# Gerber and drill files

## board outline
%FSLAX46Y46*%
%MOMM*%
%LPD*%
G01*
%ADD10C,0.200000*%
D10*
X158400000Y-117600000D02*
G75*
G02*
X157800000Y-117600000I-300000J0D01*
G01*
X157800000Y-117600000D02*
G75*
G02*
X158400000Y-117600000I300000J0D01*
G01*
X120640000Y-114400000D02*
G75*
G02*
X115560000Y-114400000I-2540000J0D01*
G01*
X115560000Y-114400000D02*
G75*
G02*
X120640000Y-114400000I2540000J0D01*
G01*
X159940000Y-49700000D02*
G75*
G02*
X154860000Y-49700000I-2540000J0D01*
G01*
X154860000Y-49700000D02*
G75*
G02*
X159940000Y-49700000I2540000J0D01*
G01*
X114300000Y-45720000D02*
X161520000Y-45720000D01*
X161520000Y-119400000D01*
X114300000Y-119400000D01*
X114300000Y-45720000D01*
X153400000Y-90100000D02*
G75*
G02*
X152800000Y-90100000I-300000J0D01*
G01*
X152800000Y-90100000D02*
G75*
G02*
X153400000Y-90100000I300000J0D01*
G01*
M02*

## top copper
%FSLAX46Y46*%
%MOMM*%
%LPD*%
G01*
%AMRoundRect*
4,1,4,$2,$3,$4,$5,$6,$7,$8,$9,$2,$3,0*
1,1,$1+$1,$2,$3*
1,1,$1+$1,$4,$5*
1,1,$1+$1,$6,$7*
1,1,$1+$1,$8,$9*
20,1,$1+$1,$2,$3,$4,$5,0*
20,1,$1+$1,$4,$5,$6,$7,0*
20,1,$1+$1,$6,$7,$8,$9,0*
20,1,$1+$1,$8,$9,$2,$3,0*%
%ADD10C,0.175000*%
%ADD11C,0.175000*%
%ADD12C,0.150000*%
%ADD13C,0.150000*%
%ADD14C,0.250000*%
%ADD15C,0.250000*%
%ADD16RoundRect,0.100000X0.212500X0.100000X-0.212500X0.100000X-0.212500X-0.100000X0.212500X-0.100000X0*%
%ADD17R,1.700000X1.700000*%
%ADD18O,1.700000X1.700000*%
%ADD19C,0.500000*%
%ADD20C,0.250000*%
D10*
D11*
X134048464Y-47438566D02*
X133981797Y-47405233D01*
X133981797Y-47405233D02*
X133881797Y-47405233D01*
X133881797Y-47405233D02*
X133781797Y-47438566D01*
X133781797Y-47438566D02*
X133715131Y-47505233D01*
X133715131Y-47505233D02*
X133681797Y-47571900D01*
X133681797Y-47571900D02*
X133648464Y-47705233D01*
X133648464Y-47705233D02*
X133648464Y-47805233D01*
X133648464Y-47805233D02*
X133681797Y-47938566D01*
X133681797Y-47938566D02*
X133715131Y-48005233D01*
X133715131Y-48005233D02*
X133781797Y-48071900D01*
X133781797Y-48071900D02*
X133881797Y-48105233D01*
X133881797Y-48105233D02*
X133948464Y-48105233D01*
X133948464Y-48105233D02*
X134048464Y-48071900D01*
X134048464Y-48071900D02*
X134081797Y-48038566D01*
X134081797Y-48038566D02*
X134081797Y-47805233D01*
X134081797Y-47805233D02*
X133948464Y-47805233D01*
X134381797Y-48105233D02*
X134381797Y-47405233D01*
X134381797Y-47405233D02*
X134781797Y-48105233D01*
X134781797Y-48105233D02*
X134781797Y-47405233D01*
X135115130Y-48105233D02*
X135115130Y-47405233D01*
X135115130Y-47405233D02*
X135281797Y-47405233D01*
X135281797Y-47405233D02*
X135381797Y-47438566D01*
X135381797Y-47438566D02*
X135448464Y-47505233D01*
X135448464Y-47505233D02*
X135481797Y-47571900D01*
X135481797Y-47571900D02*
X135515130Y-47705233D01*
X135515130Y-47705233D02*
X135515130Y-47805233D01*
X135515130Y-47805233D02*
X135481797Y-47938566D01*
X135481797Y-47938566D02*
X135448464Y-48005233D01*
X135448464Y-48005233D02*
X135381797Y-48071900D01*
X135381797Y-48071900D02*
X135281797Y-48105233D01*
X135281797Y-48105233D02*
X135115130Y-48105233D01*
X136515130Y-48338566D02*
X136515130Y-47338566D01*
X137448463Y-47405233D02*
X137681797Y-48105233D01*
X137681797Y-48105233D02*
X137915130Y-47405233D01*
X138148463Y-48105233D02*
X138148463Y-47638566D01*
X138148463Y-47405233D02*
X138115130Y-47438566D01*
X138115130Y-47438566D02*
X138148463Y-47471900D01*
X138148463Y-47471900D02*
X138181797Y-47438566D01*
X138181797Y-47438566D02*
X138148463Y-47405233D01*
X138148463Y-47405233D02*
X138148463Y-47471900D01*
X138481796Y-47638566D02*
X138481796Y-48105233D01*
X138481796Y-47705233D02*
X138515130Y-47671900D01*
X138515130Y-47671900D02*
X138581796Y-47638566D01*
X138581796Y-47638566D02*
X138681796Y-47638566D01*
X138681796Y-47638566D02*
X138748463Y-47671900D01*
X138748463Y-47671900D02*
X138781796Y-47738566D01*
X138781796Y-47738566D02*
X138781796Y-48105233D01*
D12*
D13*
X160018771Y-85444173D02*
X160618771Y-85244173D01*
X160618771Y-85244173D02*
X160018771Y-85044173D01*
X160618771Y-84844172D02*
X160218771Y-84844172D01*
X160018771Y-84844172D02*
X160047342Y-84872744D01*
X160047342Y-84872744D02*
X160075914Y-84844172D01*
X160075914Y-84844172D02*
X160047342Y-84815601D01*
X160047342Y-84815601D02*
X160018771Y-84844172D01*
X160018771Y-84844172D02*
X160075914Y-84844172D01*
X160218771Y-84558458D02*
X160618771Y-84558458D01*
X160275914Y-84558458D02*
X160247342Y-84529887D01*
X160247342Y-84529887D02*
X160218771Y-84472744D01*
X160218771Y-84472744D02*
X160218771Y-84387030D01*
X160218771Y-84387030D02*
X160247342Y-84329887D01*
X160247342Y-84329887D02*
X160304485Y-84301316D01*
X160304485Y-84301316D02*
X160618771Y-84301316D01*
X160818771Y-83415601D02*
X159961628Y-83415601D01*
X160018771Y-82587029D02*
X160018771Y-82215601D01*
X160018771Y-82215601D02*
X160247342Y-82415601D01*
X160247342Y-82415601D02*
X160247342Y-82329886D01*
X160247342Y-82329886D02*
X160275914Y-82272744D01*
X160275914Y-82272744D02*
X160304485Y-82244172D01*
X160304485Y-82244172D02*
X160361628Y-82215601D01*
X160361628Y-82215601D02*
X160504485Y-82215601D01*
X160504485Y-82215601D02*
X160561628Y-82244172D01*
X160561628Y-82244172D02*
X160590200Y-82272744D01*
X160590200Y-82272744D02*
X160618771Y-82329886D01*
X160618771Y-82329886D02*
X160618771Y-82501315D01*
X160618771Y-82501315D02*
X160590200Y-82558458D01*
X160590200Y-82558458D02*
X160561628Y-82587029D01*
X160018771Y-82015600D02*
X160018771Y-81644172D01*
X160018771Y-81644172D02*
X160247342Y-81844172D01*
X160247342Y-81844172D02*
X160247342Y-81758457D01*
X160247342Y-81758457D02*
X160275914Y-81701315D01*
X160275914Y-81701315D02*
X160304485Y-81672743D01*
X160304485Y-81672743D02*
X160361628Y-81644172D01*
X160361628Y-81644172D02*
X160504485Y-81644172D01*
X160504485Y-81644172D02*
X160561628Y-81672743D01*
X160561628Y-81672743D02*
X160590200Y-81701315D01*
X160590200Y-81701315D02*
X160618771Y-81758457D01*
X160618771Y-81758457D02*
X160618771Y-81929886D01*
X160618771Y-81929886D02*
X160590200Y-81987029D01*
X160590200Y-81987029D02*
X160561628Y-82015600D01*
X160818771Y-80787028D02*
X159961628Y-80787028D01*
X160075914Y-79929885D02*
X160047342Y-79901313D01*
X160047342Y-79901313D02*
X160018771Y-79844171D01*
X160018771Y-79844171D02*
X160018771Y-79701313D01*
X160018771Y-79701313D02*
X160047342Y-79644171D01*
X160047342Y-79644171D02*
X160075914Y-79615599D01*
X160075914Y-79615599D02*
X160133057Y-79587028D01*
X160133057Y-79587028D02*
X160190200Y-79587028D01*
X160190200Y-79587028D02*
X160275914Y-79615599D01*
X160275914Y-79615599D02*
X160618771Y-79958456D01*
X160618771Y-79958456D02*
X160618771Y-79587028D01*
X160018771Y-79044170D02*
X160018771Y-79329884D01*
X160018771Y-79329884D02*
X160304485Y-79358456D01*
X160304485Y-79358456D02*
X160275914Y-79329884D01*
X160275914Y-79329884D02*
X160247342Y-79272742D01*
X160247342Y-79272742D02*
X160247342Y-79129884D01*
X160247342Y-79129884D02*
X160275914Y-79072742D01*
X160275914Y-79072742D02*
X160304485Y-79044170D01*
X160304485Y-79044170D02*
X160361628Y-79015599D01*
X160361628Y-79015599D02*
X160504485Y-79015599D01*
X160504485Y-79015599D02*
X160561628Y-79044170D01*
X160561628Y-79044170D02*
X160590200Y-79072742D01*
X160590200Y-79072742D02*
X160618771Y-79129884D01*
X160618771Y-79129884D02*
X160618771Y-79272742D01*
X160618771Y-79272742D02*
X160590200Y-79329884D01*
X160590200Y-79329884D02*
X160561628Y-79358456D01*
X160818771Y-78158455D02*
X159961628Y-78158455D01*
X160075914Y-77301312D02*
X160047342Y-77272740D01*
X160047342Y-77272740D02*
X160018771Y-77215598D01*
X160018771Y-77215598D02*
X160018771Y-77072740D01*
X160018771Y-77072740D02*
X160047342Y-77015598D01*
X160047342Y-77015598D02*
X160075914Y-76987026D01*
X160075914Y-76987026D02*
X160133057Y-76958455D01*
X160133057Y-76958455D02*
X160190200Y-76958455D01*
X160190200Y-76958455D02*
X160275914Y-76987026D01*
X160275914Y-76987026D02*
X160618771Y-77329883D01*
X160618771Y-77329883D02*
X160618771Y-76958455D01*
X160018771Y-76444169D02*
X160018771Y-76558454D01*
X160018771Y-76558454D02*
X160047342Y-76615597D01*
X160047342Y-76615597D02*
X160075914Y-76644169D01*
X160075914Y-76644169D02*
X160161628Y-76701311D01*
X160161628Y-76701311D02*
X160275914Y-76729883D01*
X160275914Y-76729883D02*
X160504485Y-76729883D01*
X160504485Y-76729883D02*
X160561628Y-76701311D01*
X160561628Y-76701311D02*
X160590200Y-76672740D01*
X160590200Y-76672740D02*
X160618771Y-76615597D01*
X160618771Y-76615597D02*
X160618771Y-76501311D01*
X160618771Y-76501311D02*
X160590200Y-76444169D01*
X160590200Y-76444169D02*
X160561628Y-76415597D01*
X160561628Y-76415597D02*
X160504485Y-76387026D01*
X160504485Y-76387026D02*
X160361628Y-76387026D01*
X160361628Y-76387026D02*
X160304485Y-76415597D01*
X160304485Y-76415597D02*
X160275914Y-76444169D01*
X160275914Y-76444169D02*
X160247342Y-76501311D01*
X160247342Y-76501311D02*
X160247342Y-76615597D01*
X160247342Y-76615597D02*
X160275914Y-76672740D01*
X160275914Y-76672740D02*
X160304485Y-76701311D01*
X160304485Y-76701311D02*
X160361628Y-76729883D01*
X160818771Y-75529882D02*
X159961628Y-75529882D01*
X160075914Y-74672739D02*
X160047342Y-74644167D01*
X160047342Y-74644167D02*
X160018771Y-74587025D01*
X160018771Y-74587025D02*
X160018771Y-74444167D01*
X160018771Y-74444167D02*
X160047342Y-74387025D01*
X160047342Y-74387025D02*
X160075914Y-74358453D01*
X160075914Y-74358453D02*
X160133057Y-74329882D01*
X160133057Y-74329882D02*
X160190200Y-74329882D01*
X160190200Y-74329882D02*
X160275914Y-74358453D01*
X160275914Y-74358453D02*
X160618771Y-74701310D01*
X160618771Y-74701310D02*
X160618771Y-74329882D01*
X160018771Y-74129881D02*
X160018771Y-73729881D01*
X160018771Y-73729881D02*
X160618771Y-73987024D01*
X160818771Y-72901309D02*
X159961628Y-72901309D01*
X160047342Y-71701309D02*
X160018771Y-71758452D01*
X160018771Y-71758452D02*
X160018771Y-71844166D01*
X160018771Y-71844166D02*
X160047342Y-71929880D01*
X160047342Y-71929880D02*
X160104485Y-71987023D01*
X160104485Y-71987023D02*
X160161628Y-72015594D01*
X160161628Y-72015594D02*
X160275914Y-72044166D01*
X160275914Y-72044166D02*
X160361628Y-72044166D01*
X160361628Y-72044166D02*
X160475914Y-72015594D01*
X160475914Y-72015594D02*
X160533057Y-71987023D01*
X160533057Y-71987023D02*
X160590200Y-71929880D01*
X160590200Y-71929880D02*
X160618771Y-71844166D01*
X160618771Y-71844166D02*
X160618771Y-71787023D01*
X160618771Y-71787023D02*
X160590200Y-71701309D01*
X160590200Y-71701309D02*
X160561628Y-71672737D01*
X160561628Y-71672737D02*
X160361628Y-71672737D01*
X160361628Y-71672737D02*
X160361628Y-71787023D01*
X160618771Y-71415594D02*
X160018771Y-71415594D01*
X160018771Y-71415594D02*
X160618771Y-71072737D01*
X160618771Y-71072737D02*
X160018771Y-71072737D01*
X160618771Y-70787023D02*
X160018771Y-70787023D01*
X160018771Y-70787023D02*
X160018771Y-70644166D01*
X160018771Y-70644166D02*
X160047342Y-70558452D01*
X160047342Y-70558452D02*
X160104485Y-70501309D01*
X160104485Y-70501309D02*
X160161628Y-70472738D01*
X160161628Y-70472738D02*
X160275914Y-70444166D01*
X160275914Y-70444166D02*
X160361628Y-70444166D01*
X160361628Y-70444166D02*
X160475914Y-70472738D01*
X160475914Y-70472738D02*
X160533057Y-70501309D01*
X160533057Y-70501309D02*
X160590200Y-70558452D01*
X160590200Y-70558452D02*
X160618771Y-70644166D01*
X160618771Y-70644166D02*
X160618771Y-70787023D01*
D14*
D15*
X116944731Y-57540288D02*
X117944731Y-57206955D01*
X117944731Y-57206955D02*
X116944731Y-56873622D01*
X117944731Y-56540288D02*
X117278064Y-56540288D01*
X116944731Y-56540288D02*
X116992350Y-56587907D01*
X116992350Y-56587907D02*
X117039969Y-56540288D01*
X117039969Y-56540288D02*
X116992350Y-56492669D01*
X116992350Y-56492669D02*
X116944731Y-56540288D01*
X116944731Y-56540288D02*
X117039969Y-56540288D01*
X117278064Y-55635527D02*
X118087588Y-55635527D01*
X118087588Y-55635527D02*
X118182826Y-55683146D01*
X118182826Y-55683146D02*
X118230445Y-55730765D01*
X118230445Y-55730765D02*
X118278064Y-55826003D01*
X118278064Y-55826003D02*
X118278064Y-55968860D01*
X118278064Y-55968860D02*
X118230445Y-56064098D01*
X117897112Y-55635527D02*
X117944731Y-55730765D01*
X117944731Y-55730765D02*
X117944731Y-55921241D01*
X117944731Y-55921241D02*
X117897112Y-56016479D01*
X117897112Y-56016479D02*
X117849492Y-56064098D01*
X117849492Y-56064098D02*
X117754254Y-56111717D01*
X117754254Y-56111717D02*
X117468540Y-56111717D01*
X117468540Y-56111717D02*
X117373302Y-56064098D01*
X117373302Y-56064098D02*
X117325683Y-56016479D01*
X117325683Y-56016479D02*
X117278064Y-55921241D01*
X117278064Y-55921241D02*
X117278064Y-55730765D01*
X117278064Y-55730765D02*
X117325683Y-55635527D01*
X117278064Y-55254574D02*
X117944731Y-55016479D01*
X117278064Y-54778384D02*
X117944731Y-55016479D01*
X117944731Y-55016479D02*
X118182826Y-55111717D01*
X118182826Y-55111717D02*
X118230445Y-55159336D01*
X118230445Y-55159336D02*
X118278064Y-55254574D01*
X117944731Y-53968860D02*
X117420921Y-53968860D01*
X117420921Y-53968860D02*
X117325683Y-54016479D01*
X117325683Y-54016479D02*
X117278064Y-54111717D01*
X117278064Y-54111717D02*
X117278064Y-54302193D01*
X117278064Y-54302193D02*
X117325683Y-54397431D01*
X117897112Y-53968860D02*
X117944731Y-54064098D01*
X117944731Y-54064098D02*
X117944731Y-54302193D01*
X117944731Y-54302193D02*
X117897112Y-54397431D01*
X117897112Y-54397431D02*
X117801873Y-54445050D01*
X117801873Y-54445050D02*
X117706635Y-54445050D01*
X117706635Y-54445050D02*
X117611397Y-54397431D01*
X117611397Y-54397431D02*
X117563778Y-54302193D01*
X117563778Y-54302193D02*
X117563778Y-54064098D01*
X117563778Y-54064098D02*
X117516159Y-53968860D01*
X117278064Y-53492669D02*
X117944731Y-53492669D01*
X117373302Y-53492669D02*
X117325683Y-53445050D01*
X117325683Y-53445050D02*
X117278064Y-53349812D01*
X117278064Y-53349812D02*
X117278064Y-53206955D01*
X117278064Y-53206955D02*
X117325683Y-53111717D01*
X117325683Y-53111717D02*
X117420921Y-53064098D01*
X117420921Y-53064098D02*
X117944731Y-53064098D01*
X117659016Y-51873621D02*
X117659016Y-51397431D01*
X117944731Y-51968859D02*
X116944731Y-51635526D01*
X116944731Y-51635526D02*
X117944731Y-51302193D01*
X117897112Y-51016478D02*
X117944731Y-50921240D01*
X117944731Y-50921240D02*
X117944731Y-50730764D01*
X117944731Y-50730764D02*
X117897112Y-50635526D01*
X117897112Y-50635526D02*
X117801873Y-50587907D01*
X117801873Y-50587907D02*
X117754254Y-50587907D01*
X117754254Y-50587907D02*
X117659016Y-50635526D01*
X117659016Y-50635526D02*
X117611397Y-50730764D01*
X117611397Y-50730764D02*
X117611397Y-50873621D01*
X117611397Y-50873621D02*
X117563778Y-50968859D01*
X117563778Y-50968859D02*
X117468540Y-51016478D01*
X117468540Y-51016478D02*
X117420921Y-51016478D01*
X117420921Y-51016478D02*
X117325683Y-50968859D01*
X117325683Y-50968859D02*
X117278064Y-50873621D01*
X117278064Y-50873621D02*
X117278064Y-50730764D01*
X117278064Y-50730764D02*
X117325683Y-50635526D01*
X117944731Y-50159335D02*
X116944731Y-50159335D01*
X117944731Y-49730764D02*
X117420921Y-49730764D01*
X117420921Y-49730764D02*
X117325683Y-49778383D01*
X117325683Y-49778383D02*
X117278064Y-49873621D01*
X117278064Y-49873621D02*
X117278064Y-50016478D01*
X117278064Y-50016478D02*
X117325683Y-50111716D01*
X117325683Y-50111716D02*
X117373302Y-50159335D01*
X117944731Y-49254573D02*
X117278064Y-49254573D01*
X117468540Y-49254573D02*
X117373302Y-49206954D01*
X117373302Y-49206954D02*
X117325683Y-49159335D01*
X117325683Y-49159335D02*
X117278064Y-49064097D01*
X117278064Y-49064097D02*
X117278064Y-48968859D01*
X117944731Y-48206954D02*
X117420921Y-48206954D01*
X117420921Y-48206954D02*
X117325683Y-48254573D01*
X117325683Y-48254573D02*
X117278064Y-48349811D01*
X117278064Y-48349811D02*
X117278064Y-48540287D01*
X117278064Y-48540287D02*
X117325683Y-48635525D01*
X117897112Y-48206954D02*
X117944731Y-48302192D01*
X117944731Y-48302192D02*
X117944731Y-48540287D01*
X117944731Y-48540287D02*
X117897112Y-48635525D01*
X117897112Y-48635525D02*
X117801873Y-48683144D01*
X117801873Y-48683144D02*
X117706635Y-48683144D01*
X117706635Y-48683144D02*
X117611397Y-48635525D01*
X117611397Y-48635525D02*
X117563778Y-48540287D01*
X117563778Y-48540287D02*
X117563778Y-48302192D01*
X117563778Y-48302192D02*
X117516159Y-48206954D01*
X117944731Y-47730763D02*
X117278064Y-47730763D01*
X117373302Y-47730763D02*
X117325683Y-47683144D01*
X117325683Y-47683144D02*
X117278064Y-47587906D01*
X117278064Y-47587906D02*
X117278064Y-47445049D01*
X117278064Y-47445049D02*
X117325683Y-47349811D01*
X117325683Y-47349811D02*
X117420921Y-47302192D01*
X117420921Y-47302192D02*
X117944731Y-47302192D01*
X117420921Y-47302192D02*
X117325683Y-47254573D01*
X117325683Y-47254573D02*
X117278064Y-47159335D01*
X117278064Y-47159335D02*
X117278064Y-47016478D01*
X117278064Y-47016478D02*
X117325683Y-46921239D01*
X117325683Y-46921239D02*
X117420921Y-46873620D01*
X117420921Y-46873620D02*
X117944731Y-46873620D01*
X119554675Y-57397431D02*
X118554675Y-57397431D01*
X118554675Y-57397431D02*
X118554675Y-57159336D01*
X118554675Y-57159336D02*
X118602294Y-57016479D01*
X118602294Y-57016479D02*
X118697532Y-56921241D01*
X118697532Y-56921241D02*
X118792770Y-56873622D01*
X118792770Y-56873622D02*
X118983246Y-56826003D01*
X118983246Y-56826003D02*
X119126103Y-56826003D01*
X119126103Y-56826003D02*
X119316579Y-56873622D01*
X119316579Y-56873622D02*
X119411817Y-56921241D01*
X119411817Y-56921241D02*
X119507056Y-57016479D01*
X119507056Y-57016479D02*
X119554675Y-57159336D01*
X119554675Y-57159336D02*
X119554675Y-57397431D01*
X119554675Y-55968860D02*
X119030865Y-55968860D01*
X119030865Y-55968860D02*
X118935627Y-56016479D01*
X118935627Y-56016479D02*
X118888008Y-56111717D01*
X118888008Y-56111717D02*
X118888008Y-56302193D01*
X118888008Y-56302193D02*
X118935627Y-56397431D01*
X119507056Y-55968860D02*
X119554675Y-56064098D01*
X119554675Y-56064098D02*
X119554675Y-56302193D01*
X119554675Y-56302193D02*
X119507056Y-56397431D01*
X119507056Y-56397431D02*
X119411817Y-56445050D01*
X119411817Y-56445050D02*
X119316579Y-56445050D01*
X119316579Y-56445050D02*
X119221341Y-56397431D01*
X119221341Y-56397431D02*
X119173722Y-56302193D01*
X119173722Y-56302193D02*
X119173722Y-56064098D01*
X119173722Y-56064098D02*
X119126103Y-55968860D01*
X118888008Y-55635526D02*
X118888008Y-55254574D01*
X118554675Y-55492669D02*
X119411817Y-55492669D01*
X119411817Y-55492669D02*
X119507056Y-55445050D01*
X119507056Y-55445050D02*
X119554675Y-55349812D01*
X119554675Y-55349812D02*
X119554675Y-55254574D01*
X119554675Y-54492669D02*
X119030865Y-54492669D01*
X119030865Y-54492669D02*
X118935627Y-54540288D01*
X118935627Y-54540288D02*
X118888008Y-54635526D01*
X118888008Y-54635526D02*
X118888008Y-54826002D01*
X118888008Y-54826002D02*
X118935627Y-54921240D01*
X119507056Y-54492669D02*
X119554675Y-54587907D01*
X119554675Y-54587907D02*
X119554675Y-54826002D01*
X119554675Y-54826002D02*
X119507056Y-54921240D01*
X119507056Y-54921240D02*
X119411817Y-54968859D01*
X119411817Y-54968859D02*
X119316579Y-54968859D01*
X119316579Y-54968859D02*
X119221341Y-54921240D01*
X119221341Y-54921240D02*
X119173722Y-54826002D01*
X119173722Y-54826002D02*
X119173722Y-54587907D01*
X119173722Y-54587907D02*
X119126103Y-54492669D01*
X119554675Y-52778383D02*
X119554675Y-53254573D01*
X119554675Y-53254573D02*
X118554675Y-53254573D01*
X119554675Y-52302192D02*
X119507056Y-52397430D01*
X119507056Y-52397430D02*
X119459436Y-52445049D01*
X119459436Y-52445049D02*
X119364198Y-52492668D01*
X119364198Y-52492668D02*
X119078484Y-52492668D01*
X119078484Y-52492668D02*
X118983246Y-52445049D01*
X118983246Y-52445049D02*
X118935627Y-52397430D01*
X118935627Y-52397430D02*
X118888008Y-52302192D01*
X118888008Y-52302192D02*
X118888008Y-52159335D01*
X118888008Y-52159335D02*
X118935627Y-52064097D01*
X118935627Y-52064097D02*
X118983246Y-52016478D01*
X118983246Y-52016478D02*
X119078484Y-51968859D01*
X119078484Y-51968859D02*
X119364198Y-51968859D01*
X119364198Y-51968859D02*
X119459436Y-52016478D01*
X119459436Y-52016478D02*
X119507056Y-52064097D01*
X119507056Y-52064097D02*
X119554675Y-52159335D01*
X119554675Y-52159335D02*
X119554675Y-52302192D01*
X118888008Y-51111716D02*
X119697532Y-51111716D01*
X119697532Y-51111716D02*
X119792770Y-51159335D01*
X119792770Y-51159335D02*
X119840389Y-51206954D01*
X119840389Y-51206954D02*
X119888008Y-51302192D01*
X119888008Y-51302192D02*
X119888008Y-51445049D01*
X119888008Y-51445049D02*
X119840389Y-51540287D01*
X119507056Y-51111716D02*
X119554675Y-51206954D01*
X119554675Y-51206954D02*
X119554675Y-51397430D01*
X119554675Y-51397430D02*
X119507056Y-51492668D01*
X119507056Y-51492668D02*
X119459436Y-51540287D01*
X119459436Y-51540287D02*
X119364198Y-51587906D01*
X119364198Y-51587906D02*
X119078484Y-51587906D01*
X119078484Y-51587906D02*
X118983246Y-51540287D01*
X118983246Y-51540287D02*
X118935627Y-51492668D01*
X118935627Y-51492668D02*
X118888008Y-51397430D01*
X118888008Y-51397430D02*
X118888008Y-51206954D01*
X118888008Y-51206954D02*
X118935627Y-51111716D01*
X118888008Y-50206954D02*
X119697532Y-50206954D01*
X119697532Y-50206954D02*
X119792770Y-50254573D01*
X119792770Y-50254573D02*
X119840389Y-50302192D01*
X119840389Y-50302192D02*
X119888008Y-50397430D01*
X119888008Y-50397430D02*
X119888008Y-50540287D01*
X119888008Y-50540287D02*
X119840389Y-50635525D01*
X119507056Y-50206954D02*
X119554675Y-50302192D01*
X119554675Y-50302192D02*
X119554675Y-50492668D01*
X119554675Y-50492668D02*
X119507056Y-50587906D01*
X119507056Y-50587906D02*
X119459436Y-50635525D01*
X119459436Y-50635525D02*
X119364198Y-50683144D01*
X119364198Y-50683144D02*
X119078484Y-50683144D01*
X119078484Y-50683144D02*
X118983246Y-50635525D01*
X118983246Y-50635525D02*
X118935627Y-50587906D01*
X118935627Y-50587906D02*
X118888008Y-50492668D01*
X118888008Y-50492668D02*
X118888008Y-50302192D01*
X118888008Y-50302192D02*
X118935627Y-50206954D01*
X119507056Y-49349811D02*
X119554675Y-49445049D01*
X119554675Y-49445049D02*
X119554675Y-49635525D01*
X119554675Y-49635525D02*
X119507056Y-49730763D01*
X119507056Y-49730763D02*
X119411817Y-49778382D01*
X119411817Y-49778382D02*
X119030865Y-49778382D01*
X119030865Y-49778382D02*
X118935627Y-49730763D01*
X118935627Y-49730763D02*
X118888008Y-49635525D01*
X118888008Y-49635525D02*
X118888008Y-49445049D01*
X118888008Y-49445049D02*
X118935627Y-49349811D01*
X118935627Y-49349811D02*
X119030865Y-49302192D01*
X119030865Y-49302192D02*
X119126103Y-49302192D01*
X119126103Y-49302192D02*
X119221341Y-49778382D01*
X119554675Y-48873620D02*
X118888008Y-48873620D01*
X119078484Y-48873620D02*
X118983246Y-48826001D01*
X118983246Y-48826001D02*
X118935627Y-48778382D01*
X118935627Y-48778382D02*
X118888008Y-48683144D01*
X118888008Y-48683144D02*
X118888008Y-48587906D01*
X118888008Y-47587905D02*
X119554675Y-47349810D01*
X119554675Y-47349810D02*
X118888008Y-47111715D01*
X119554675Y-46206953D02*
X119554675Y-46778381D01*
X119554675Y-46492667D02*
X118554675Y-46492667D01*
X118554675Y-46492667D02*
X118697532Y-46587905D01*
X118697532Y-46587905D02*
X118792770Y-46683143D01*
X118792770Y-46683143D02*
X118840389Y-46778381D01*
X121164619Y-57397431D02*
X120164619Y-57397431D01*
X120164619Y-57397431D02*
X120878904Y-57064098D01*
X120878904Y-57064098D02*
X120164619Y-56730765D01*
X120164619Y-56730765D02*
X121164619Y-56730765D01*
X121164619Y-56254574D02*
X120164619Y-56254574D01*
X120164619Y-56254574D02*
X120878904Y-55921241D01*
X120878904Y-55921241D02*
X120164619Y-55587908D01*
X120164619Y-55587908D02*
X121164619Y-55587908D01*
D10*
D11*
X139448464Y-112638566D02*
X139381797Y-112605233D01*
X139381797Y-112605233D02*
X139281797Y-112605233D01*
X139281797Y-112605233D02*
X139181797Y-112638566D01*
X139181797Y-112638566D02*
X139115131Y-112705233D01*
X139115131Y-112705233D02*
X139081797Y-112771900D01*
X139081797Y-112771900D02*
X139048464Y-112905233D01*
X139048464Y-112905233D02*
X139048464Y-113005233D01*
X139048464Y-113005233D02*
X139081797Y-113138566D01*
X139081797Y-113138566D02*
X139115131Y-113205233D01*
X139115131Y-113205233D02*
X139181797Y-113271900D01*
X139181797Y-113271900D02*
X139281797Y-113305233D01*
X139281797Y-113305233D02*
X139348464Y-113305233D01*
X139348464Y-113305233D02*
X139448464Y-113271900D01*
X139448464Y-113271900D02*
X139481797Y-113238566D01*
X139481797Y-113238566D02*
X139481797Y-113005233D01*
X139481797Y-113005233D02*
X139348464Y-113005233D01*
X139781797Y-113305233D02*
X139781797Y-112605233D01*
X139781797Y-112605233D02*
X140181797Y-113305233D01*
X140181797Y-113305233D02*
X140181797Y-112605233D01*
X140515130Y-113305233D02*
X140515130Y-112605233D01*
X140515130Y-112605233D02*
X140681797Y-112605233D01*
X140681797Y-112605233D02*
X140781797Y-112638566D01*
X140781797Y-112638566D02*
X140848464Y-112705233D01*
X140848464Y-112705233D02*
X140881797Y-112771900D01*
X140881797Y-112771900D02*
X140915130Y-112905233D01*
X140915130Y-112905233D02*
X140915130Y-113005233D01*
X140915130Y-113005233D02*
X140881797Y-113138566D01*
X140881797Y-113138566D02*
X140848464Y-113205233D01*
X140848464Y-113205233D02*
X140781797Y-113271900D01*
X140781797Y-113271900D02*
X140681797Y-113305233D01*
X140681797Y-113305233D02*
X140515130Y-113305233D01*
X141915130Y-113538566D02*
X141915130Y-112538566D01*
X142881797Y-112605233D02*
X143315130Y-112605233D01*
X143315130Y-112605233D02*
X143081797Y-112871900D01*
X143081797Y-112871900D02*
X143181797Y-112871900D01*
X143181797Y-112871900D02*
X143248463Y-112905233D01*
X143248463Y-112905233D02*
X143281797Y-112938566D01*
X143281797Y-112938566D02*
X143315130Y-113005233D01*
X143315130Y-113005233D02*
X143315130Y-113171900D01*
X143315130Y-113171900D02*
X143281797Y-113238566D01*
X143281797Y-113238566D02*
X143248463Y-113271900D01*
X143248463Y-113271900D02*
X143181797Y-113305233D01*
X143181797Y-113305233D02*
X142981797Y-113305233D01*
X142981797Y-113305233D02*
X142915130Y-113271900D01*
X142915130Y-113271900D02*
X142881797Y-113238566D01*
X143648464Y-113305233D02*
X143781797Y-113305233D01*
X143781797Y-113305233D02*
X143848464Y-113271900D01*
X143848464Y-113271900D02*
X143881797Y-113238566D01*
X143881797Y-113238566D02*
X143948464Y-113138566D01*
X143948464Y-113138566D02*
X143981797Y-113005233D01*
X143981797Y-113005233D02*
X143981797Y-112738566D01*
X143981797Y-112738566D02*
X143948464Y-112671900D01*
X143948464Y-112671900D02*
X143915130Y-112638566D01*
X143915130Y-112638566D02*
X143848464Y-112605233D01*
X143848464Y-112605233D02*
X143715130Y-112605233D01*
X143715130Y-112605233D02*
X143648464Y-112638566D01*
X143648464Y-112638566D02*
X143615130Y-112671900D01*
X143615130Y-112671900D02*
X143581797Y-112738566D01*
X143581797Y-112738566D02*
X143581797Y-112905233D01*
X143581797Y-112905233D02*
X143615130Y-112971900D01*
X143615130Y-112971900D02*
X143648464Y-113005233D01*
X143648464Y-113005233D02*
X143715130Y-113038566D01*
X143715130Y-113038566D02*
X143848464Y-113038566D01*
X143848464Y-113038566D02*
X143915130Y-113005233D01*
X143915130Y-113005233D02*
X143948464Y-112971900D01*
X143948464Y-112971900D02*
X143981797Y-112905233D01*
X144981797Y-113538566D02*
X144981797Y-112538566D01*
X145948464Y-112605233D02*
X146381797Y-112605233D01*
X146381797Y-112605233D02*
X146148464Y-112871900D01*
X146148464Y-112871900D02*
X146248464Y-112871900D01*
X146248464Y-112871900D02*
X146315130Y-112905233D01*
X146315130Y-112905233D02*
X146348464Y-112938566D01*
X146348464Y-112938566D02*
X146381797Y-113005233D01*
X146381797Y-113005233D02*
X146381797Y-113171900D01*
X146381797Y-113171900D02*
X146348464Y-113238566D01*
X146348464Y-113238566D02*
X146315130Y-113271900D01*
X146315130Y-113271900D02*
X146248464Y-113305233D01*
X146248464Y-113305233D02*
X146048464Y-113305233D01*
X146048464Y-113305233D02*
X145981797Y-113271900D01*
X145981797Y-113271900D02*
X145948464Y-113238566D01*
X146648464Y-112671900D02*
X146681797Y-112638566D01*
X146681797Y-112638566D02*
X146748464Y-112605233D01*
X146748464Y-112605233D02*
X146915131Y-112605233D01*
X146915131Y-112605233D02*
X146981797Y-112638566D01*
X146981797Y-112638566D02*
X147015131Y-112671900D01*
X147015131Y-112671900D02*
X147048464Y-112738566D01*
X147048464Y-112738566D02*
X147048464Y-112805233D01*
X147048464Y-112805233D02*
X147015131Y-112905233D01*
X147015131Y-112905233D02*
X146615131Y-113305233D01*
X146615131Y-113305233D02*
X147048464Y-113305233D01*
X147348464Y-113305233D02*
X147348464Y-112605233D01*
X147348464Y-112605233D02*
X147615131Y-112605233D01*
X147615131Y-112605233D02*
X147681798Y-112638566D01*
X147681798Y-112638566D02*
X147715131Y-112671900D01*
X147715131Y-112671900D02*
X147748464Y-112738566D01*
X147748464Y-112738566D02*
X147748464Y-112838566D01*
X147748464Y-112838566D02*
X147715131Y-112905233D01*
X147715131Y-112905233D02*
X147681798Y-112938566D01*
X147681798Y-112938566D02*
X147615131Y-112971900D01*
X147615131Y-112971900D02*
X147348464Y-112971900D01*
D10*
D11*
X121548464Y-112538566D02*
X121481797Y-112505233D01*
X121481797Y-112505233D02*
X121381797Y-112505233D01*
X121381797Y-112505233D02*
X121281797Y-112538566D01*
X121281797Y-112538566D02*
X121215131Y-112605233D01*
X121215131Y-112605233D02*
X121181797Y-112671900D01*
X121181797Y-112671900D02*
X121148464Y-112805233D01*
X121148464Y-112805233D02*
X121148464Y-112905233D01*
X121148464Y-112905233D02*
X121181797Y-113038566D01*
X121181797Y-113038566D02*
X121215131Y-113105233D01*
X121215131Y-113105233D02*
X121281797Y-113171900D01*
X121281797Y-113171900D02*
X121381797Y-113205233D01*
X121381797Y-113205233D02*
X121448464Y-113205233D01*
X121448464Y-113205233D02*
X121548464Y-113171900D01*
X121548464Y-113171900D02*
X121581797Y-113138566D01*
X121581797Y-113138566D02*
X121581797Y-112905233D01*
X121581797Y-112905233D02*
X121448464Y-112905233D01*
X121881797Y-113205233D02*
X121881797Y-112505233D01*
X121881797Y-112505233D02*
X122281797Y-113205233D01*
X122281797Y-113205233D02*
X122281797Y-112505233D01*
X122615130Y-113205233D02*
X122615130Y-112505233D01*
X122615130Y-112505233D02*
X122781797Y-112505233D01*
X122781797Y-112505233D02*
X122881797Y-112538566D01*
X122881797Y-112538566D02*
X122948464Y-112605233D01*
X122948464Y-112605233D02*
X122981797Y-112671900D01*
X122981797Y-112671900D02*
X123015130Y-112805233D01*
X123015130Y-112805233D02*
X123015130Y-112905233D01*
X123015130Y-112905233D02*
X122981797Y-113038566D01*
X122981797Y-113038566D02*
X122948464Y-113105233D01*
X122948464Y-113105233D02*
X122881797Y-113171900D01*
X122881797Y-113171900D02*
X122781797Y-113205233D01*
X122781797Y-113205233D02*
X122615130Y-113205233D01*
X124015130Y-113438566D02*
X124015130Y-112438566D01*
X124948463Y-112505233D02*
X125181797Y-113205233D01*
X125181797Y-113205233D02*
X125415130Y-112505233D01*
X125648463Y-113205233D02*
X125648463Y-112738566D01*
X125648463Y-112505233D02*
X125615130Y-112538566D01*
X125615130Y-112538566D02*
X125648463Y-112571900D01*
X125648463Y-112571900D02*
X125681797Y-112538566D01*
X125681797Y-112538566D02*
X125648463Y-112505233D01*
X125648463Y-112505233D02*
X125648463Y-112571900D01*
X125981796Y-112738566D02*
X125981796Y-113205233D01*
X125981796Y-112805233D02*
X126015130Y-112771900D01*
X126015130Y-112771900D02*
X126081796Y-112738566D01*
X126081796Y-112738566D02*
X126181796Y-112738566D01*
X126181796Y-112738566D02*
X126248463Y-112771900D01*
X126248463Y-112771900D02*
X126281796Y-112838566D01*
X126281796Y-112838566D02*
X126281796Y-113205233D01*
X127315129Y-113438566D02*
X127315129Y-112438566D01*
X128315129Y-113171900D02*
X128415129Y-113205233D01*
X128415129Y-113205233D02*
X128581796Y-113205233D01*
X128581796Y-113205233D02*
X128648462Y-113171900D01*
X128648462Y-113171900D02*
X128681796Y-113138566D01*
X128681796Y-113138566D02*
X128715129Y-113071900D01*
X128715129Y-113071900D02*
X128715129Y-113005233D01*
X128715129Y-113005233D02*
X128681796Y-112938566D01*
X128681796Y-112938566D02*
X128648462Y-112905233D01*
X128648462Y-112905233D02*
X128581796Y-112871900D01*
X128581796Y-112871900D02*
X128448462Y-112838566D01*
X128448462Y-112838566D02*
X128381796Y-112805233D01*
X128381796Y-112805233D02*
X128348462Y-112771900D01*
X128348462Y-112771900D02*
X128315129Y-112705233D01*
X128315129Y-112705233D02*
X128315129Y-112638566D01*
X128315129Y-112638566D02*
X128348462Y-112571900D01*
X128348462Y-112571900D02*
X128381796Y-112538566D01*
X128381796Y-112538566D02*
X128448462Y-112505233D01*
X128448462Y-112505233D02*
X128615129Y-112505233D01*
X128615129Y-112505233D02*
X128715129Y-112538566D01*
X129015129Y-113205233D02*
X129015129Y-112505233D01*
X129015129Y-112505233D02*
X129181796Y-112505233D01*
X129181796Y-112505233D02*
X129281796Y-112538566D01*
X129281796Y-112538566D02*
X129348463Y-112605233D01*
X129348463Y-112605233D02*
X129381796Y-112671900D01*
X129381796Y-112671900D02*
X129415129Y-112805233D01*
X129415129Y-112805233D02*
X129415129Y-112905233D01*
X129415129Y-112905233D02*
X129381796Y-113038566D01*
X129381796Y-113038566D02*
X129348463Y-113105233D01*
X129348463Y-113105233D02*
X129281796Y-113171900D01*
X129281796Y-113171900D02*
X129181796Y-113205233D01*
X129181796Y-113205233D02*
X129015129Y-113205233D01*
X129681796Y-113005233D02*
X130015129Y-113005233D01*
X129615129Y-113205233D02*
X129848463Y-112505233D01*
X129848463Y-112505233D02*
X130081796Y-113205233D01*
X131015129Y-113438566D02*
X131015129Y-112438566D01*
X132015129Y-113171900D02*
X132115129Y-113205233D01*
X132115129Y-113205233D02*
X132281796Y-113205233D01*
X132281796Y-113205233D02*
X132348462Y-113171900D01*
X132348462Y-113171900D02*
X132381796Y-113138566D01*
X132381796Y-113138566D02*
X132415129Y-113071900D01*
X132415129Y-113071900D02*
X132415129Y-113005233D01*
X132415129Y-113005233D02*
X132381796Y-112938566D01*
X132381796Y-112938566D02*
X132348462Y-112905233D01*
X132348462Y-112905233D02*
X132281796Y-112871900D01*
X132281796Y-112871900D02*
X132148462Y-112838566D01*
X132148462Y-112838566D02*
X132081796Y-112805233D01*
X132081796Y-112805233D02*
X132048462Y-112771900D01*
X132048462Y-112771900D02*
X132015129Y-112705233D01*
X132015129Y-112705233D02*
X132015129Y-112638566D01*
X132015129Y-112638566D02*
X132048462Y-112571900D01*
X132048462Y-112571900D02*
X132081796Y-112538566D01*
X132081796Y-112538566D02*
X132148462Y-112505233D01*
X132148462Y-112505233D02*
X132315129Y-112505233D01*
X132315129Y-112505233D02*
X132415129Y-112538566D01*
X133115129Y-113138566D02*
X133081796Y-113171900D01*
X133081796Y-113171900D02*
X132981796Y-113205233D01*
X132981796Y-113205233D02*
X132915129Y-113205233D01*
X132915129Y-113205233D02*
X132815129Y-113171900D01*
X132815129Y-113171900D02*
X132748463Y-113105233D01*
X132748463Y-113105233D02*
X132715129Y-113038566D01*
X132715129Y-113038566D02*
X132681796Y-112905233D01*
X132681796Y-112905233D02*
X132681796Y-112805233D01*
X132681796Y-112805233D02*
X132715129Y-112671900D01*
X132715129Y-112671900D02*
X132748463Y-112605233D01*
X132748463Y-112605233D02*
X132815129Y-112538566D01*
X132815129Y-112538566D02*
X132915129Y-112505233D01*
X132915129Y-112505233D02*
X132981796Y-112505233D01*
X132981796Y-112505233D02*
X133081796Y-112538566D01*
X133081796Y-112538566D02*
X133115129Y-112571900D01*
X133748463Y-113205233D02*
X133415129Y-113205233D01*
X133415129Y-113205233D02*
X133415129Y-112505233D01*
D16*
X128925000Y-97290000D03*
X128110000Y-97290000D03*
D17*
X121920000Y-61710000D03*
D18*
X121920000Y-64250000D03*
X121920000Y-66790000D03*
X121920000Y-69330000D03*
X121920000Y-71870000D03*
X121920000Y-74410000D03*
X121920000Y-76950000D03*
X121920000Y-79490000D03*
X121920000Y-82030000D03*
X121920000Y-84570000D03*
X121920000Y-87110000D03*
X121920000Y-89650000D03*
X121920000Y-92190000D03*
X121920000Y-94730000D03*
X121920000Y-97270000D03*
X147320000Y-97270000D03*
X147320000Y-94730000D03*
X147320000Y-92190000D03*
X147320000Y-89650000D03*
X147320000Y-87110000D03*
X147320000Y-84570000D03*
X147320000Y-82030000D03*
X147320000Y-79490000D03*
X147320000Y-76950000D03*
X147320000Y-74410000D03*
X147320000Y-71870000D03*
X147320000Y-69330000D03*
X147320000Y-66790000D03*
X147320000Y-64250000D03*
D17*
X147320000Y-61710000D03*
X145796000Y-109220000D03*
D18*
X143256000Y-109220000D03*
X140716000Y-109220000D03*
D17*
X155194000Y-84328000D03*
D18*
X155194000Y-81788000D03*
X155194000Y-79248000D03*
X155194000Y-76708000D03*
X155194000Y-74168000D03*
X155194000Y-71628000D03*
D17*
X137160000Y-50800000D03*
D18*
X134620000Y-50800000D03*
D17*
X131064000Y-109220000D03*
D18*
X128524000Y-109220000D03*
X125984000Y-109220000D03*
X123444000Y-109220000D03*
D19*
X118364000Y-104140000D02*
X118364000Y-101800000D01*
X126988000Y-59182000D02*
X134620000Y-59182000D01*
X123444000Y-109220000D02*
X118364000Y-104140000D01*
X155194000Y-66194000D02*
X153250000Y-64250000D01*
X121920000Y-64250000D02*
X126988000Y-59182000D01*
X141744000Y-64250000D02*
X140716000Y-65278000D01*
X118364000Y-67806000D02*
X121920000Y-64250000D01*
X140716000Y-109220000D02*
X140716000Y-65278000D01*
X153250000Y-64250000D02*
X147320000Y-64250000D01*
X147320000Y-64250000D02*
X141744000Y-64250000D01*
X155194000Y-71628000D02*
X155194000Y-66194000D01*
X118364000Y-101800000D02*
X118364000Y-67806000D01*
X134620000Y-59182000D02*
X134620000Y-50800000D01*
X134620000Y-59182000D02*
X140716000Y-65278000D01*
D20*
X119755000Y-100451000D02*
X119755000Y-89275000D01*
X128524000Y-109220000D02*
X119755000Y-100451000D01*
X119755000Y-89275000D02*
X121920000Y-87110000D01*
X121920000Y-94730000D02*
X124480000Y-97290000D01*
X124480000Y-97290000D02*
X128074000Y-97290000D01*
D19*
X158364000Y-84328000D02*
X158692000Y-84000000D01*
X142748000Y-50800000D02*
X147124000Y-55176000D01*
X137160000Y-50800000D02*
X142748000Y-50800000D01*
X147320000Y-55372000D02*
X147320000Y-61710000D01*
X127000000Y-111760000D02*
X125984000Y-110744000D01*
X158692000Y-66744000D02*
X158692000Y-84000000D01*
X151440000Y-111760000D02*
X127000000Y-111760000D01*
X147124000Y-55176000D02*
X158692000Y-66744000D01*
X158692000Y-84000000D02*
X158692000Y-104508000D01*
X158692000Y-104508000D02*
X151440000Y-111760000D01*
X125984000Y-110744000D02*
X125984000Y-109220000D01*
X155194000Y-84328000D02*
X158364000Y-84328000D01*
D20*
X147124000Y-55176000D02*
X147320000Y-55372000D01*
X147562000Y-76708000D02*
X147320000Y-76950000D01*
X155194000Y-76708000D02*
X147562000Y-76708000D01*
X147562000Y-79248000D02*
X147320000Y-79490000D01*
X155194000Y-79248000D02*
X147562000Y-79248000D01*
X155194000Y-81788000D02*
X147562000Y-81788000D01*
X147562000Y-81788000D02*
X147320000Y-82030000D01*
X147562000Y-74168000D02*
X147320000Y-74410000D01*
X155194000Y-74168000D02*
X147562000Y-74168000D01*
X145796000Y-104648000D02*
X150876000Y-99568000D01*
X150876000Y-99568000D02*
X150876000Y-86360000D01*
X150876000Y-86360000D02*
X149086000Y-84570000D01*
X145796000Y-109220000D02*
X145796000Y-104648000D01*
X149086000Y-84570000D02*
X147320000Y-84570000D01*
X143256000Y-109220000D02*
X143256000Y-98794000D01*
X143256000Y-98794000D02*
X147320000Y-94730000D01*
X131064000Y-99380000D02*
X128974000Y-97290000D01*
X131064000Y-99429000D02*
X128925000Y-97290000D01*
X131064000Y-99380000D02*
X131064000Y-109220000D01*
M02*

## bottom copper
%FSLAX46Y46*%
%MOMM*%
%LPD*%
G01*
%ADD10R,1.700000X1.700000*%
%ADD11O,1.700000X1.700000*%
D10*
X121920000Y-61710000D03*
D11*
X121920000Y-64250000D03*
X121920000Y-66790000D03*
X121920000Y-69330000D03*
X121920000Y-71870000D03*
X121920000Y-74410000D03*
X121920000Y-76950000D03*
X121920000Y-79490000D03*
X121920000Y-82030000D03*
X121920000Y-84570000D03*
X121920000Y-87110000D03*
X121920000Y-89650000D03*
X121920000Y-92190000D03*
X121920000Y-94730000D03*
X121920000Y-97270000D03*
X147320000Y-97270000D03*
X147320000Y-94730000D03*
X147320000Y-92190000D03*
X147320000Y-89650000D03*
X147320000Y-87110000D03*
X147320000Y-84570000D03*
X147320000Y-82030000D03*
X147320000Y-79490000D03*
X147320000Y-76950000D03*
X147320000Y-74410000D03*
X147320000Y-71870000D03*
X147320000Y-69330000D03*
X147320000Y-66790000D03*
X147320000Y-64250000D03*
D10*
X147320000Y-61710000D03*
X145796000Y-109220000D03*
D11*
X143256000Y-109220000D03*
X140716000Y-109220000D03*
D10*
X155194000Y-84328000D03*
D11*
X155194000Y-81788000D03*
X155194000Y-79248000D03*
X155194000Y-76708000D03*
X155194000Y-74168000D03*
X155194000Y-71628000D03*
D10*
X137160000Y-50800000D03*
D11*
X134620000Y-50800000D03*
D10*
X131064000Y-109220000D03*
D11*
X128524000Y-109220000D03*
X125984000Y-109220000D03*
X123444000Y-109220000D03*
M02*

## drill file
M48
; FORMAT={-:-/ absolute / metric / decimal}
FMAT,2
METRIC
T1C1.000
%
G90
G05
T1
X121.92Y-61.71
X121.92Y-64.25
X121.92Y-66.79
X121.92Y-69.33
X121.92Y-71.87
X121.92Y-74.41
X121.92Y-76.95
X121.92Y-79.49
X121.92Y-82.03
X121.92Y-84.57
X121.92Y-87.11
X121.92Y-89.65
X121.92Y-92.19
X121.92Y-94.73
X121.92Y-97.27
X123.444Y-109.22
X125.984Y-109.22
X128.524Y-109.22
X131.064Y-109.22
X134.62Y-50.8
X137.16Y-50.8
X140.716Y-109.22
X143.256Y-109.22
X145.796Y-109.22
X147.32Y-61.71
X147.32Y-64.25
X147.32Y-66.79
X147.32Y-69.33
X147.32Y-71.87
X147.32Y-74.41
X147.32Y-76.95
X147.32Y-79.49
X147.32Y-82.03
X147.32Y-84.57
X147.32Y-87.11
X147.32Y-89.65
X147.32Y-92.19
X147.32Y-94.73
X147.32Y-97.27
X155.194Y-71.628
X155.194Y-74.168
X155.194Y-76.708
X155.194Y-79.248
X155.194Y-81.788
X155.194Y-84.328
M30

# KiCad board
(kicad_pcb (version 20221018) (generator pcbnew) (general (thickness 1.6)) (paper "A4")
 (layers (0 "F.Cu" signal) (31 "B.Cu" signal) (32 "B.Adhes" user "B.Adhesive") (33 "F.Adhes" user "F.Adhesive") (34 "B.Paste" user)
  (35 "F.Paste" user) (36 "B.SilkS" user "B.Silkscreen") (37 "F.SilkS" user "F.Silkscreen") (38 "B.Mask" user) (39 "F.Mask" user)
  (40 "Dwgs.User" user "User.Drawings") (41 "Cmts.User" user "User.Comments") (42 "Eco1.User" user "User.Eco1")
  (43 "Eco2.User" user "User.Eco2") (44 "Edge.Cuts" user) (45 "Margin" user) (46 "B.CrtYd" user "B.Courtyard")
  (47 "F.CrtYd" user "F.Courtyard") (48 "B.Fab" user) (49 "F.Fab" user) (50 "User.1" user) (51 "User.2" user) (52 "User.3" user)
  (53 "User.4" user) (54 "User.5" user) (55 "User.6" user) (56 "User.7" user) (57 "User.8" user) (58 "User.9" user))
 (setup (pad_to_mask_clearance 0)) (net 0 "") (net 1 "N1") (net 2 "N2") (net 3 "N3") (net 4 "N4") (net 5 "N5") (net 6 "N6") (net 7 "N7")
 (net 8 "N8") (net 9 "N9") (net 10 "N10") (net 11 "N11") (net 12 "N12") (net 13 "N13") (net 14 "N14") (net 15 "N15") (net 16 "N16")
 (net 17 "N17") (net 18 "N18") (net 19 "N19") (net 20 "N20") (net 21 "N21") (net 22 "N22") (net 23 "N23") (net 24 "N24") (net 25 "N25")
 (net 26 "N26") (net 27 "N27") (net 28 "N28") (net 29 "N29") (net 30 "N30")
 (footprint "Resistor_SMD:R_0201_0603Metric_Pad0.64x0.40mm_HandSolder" (layer "F.Cu") (at 128.5175 97.29 180)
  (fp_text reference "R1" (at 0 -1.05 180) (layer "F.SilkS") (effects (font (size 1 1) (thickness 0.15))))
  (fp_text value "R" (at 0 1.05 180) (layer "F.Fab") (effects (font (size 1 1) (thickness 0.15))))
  (pad "" smd roundrect (at -0.4325 0 180) (size 0.458 0.36) (layers "F.Paste") (roundrect_rratio 0.25))
  (pad "" smd roundrect (at 0.4325 0 180) (size 0.458 0.36) (layers "F.Paste") (roundrect_rratio 0.25))
  (pad "1" smd roundrect (at -0.4075 0 180) (size 0.625 0.4) (layers "F.Cu" "F.Mask") (roundrect_rratio 0.25) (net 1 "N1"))
  (pad "2" smd roundrect (at 0.4075 0 180) (size 0.625 0.4) (layers "F.Cu" "F.Mask") (roundrect_rratio 0.25) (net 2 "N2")))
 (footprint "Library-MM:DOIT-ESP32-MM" (layer "F.Cu") (at 121.92 60.96)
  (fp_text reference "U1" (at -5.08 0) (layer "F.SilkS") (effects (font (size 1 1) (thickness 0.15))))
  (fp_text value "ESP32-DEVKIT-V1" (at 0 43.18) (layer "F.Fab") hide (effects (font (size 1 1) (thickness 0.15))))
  (pad "1" thru_hole rect (at 0 0.75) (size 1.7 1.7) (drill 1) (layers "*.Cu" "*.Mask") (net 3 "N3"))
  (pad "2" thru_hole oval (at 0 3.29) (size 1.7 1.7) (drill 1) (layers "*.Cu" "*.Mask") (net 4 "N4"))
  (pad "3" thru_hole oval (at 0 5.83) (size 1.7 1.7) (drill 1) (layers "*.Cu" "*.Mask") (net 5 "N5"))
  (pad "4" thru_hole oval (at 0 8.37) (size 1.7 1.7) (drill 1) (layers "*.Cu" "*.Mask") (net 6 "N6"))
  (pad "5" thru_hole oval (at 0 10.91) (size 1.7 1.7) (drill 1) (layers "*.Cu" "*.Mask") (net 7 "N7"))
  (pad "6" thru_hole oval (at 0 13.45) (size 1.7 1.7) (drill 1) (layers "*.Cu" "*.Mask") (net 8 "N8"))
  (pad "7" thru_hole oval (at 0 15.99) (size 1.7 1.7) (drill 1) (layers "*.Cu" "*.Mask") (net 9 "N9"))
  (pad "8" thru_hole oval (at 0 18.53) (size 1.7 1.7) (drill 1) (layers "*.Cu" "*.Mask") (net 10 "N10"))
  (pad "9" thru_hole oval (at 0 21.07) (size 1.7 1.7) (drill 1) (layers "*.Cu" "*.Mask") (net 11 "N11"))
  (pad "10" thru_hole oval (at 0 23.61) (size 1.7 1.7) (drill 1) (layers "*.Cu" "*.Mask") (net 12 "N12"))
  (pad "11" thru_hole oval (at 0 26.15) (size 1.7 1.7) (drill 1) (layers "*.Cu" "*.Mask") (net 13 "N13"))
  (pad "12" thru_hole oval (at 0 28.69) (size 1.7 1.7) (drill 1) (layers "*.Cu" "*.Mask") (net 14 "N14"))
  (pad "13" thru_hole oval (at 0 31.23) (size 1.7 1.7) (drill 1) (layers "*.Cu" "*.Mask") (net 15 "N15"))
  (pad "14" thru_hole oval (at 0 33.77) (size 1.7 1.7) (drill 1) (layers "*.Cu" "*.Mask") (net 2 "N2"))
  (pad "15" thru_hole oval (at 0 36.31) (size 1.7 1.7) (drill 1) (layers "*.Cu" "*.Mask") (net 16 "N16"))
  (pad "16" thru_hole oval (at 25.4 36.31) (size 1.7 1.7) (drill 1) (layers "*.Cu" "*.Mask") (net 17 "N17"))
  (pad "17" thru_hole oval (at 25.4 33.77) (size 1.7 1.7) (drill 1) (layers "*.Cu" "*.Mask") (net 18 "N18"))
  (pad "18" thru_hole oval (at 25.4 31.23) (size 1.7 1.7) (drill 1) (layers "*.Cu" "*.Mask") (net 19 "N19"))
  (pad "19" thru_hole oval (at 25.4 28.69) (size 1.7 1.7) (drill 1) (layers "*.Cu" "*.Mask") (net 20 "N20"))
  (pad "20" thru_hole oval (at 25.4 26.15) (size 1.7 1.7) (drill 1) (layers "*.Cu" "*.Mask") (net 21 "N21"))
  (pad "21" thru_hole oval (at 25.4 23.61) (size 1.7 1.7) (drill 1) (layers "*.Cu" "*.Mask") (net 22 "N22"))
  (pad "22" thru_hole oval (at 25.4 21.07) (size 1.7 1.7) (drill 1) (layers "*.Cu" "*.Mask") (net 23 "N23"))
  (pad "23" thru_hole oval (at 25.4 18.53) (size 1.7 1.7) (drill 1) (layers "*.Cu" "*.Mask") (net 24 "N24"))
  (pad "24" thru_hole oval (at 25.4 15.99) (size 1.7 1.7) (drill 1) (layers "*.Cu" "*.Mask") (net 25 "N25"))
  (pad "25" thru_hole oval (at 25.4 13.45) (size 1.7 1.7) (drill 1) (layers "*.Cu" "*.Mask") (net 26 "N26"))
  (pad "26" thru_hole oval (at 25.4 10.91) (size 1.7 1.7) (drill 1) (layers "*.Cu" "*.Mask") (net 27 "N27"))
  (pad "27" thru_hole oval (at 25.4 8.37) (size 1.7 1.7) (drill 1) (layers "*.Cu" "*.Mask") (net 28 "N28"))
  (pad "28" thru_hole oval (at 25.4 5.83) (size 1.7 1.7) (drill 1) (layers "*.Cu" "*.Mask") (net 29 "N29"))
  (pad "29" thru_hole oval (at 25.4 3.29) (size 1.7 1.7) (drill 1) (layers "*.Cu" "*.Mask") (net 4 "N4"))
  (pad "30" thru_hole rect (at 25.4 0.75) (size 1.7 1.7) (drill 1) (layers "*.Cu" "*.Mask") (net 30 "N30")))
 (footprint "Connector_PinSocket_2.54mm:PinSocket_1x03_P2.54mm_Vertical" (layer "F.Cu") (at 145.796 109.22 -90)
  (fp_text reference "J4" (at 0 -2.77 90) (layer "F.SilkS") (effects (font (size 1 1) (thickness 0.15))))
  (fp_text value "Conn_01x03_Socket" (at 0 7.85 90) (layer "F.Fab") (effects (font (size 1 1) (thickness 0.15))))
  (pad "1" thru_hole rect (at 0 0 270) (size 1.7 1.7) (drill 1) (layers "*.Cu" "*.Mask") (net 22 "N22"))
  (pad "2" thru_hole oval (at 0 2.54 270) (size 1.7 1.7) (drill 1) (layers "*.Cu" "*.Mask") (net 18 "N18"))
  (pad "3" thru_hole oval (at 0 5.08 270) (size 1.7 1.7) (drill 1) (layers "*.Cu" "*.Mask") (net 4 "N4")))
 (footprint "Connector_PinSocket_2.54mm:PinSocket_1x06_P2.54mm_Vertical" (layer "F.Cu") (at 155.194 84.328 180)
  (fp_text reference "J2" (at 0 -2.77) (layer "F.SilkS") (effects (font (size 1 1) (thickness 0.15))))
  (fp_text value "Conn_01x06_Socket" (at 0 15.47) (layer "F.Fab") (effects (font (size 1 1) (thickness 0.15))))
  (pad "1" thru_hole rect (at 0 0 180) (size 1.7 1.7) (drill 1) (layers "*.Cu" "*.Mask") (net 30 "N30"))
  (pad "2" thru_hole oval (at 0 2.54 180) (size 1.7 1.7) (drill 1) (layers "*.Cu" "*.Mask") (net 23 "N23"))
  (pad "3" thru_hole oval (at 0 5.08 180) (size 1.7 1.7) (drill 1) (layers "*.Cu" "*.Mask") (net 24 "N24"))
  (pad "4" thru_hole oval (at 0 7.62 180) (size 1.7 1.7) (drill 1) (layers "*.Cu" "*.Mask") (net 25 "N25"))
  (pad "5" thru_hole oval (at 0 10.16 180) (size 1.7 1.7) (drill 1) (layers "*.Cu" "*.Mask") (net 26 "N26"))
  (pad "6" thru_hole oval (at 0 12.7 180) (size 1.7 1.7) (drill 1) (layers "*.Cu" "*.Mask") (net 4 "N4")))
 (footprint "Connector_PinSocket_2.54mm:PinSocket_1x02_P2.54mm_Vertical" (layer "F.Cu") (at 137.16 50.8 -90)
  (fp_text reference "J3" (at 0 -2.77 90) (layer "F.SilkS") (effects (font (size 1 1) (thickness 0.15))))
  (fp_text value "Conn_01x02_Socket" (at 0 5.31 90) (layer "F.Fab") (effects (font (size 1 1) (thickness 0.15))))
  (pad "1" thru_hole rect (at 0 0 270) (size 1.7 1.7) (drill 1) (layers "*.Cu" "*.Mask") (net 30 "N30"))
  (pad "2" thru_hole oval (at 0 2.54 270) (size 1.7 1.7) (drill 1) (layers "*.Cu" "*.Mask") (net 4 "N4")))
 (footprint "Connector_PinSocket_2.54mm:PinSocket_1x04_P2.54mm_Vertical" (layer "F.Cu") (at 131.064 109.22 -90)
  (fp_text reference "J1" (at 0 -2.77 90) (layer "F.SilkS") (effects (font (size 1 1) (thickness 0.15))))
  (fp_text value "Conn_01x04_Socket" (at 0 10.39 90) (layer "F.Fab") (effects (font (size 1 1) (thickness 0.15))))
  (pad "1" thru_hole rect (at 0 0 270) (size 1.7 1.7) (drill 1) (layers "*.Cu" "*.Mask") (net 1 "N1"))
  (pad "2" thru_hole oval (at 0 2.54 270) (size 1.7 1.7) (drill 1) (layers "*.Cu" "*.Mask") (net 13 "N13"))
  (pad "3" thru_hole oval (at 0 5.08 270) (size 1.7 1.7) (drill 1) (layers "*.Cu" "*.Mask") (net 30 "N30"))
  (pad "4" thru_hole oval (at 0 7.62 270) (size 1.7 1.7) (drill 1) (layers "*.Cu" "*.Mask") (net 4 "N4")))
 (gr_circle (center 158.1 117.6) (end 158.4 117.6) (stroke (width 0.2) (type default)) (fill none) (layer "Edge.Cuts"))
 (gr_circle (center 118.1 114.4) (end 120.64 114.4) (stroke (width 0.2) (type default)) (fill none) (layer "Edge.Cuts"))
 (gr_circle (center 157.4 49.7) (end 159.94 49.7) (stroke (width 0.2) (type solid)) (fill none) (layer "Edge.Cuts"))
 (gr_rect (start 114.3 45.72) (end 161.52 119.4) (stroke (width 0.2) (type default)) (fill none) (layer "Edge.Cuts"))
 (gr_circle (center 153.1 90.1) (end 153.4 90.1) (stroke (width 0.2) (type default)) (fill none) (layer "Edge.Cuts"))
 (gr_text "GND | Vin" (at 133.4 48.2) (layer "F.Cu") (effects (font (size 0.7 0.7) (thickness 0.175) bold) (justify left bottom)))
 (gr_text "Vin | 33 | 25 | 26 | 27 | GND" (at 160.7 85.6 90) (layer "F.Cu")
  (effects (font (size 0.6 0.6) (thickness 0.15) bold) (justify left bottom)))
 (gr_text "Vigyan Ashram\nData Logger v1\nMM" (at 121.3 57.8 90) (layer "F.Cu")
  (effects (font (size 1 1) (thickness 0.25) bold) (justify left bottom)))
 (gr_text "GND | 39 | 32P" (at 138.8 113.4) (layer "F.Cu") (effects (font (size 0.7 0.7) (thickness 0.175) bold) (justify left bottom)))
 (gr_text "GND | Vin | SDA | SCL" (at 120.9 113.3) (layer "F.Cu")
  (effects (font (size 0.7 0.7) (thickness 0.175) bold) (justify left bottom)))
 (segment (start 118.364 104.14) (end 118.364 101.8) (width 0.5) (layer "F.Cu") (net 4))
 (segment (start 126.988 59.182) (end 134.62 59.182) (width 0.5) (layer "F.Cu") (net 4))
 (segment (start 123.444 109.22) (end 118.364 104.14) (width 0.5) (layer "F.Cu") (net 4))
 (segment (start 155.194 66.194) (end 153.25 64.25) (width 0.5) (layer "F.Cu") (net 4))
 (segment (start 121.92 64.25) (end 126.988 59.182) (width 0.5) (layer "F.Cu") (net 4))
 (segment (start 141.744 64.25) (end 140.716 65.278) (width 0.5) (layer "F.Cu") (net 4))
 (segment (start 118.364 67.806) (end 121.92 64.25) (width 0.5) (layer "F.Cu") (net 4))
 (segment (start 140.716 109.22) (end 140.716 65.278) (width 0.5) (layer "F.Cu") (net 4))
 (segment (start 153.25 64.25) (end 147.32 64.25) (width 0.5) (layer "F.Cu") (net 4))
 (segment (start 147.32 64.25) (end 141.744 64.25) (width 0.5) (layer "F.Cu") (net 4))
 (segment (start 155.194 71.628) (end 155.194 66.194) (width 0.5) (layer "F.Cu") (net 4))
 (segment (start 118.364 101.8) (end 118.364 67.806) (width 0.5) (layer "F.Cu") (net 4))
 (segment (start 134.62 59.182) (end 134.62 50.8) (width 0.5) (layer "F.Cu") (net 4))
 (segment (start 134.62 59.182) (end 140.716 65.278) (width 0.5) (layer "F.Cu") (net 4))
 (segment (start 119.755 100.451) (end 119.755 89.275) (width 0.25) (layer "F.Cu") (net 13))
 (segment (start 128.524 109.22) (end 119.755 100.451) (width 0.25) (layer "F.Cu") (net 13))
 (segment (start 119.755 89.275) (end 121.92 87.11) (width 0.25) (layer "F.Cu") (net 13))
 (segment (start 121.92 94.73) (end 124.48 97.29) (width 0.25) (layer "F.Cu") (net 2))
 (segment (start 124.48 97.29) (end 128.074 97.29) (width 0.25) (layer "F.Cu") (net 2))
 (segment (start 158.364 84.328) (end 158.692 84) (width 0.5) (layer "F.Cu") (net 30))
 (segment (start 142.748 50.8) (end 147.124 55.176) (width 0.5) (layer "F.Cu") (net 30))
 (segment (start 137.16 50.8) (end 142.748 50.8) (width 0.5) (layer "F.Cu") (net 30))
 (segment (start 147.32 55.372) (end 147.32 61.71) (width 0.5) (layer "F.Cu") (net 30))
 (segment (start 127 111.76) (end 125.984 110.744) (width 0.5) (layer "F.Cu") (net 30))
 (segment (start 158.692 66.744) (end 158.692 84) (width 0.5) (layer "F.Cu") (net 30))
 (segment (start 151.44 111.76) (end 127 111.76) (width 0.5) (layer "F.Cu") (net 30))
 (segment (start 147.124 55.176) (end 158.692 66.744) (width 0.5) (layer "F.Cu") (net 30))
 (segment (start 158.692 84) (end 158.692 104.508) (width 0.5) (layer "F.Cu") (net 30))
 (segment (start 158.692 104.508) (end 151.44 111.76) (width 0.5) (layer "F.Cu") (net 30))
 (segment (start 125.984 110.744) (end 125.984 109.22) (width 0.5) (layer "F.Cu") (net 30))
 (segment (start 155.194 84.328) (end 158.364 84.328) (width 0.5) (layer "F.Cu") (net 30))
 (segment (start 147.124 55.176) (end 147.32 55.372) (width 0.25) (layer "F.Cu") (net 30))
 (segment (start 147.562 76.708) (end 147.32 76.95) (width 0.25) (layer "F.Cu") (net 25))
 (segment (start 155.194 76.708) (end 147.562 76.708) (width 0.25) (layer "F.Cu") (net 25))
 (segment (start 147.562 79.248) (end 147.32 79.49) (width 0.25) (layer "F.Cu") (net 24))
 (segment (start 155.194 79.248) (end 147.562 79.248) (width 0.25) (layer "F.Cu") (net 24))
 (segment (start 155.194 81.788) (end 147.562 81.788) (width 0.25) (layer "F.Cu") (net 23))
 (segment (start 147.562 81.788) (end 147.32 82.03) (width 0.25) (layer "F.Cu") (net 23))
 (segment (start 147.562 74.168) (end 147.32 74.41) (width 0.25) (layer "F.Cu") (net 26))
 (segment (start 155.194 74.168) (end 147.562 74.168) (width 0.25) (layer "F.Cu") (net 26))
 (segment (start 145.796 104.648) (end 150.876 99.568) (width 0.25) (layer "F.Cu") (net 22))
 (segment (start 150.876 99.568) (end 150.876 86.36) (width 0.25) (layer "F.Cu") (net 22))
 (segment (start 150.876 86.36) (end 149.086 84.57) (width 0.25) (layer "F.Cu") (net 22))
 (segment (start 145.796 109.22) (end 145.796 104.648) (width 0.25) (layer "F.Cu") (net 22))
 (segment (start 149.086 84.57) (end 147.32 84.57) (width 0.25) (layer "F.Cu") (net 22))
 (segment (start 143.256 109.22) (end 143.256 98.794) (width 0.25) (layer "F.Cu") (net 18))
 (segment (start 143.256 98.794) (end 147.32 94.73) (width 0.25) (layer "F.Cu") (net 18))
 (segment (start 131.064 99.38) (end 128.974 97.29) (width 0.25) (layer "F.Cu") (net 1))
 (segment (start 131.064 99.429) (end 128.925 97.29) (width 0.25) (layer "F.Cu") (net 1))
 (segment (start 131.064 99.38) (end 131.064 109.22) (width 0.25) (layer "F.Cu") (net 1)))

